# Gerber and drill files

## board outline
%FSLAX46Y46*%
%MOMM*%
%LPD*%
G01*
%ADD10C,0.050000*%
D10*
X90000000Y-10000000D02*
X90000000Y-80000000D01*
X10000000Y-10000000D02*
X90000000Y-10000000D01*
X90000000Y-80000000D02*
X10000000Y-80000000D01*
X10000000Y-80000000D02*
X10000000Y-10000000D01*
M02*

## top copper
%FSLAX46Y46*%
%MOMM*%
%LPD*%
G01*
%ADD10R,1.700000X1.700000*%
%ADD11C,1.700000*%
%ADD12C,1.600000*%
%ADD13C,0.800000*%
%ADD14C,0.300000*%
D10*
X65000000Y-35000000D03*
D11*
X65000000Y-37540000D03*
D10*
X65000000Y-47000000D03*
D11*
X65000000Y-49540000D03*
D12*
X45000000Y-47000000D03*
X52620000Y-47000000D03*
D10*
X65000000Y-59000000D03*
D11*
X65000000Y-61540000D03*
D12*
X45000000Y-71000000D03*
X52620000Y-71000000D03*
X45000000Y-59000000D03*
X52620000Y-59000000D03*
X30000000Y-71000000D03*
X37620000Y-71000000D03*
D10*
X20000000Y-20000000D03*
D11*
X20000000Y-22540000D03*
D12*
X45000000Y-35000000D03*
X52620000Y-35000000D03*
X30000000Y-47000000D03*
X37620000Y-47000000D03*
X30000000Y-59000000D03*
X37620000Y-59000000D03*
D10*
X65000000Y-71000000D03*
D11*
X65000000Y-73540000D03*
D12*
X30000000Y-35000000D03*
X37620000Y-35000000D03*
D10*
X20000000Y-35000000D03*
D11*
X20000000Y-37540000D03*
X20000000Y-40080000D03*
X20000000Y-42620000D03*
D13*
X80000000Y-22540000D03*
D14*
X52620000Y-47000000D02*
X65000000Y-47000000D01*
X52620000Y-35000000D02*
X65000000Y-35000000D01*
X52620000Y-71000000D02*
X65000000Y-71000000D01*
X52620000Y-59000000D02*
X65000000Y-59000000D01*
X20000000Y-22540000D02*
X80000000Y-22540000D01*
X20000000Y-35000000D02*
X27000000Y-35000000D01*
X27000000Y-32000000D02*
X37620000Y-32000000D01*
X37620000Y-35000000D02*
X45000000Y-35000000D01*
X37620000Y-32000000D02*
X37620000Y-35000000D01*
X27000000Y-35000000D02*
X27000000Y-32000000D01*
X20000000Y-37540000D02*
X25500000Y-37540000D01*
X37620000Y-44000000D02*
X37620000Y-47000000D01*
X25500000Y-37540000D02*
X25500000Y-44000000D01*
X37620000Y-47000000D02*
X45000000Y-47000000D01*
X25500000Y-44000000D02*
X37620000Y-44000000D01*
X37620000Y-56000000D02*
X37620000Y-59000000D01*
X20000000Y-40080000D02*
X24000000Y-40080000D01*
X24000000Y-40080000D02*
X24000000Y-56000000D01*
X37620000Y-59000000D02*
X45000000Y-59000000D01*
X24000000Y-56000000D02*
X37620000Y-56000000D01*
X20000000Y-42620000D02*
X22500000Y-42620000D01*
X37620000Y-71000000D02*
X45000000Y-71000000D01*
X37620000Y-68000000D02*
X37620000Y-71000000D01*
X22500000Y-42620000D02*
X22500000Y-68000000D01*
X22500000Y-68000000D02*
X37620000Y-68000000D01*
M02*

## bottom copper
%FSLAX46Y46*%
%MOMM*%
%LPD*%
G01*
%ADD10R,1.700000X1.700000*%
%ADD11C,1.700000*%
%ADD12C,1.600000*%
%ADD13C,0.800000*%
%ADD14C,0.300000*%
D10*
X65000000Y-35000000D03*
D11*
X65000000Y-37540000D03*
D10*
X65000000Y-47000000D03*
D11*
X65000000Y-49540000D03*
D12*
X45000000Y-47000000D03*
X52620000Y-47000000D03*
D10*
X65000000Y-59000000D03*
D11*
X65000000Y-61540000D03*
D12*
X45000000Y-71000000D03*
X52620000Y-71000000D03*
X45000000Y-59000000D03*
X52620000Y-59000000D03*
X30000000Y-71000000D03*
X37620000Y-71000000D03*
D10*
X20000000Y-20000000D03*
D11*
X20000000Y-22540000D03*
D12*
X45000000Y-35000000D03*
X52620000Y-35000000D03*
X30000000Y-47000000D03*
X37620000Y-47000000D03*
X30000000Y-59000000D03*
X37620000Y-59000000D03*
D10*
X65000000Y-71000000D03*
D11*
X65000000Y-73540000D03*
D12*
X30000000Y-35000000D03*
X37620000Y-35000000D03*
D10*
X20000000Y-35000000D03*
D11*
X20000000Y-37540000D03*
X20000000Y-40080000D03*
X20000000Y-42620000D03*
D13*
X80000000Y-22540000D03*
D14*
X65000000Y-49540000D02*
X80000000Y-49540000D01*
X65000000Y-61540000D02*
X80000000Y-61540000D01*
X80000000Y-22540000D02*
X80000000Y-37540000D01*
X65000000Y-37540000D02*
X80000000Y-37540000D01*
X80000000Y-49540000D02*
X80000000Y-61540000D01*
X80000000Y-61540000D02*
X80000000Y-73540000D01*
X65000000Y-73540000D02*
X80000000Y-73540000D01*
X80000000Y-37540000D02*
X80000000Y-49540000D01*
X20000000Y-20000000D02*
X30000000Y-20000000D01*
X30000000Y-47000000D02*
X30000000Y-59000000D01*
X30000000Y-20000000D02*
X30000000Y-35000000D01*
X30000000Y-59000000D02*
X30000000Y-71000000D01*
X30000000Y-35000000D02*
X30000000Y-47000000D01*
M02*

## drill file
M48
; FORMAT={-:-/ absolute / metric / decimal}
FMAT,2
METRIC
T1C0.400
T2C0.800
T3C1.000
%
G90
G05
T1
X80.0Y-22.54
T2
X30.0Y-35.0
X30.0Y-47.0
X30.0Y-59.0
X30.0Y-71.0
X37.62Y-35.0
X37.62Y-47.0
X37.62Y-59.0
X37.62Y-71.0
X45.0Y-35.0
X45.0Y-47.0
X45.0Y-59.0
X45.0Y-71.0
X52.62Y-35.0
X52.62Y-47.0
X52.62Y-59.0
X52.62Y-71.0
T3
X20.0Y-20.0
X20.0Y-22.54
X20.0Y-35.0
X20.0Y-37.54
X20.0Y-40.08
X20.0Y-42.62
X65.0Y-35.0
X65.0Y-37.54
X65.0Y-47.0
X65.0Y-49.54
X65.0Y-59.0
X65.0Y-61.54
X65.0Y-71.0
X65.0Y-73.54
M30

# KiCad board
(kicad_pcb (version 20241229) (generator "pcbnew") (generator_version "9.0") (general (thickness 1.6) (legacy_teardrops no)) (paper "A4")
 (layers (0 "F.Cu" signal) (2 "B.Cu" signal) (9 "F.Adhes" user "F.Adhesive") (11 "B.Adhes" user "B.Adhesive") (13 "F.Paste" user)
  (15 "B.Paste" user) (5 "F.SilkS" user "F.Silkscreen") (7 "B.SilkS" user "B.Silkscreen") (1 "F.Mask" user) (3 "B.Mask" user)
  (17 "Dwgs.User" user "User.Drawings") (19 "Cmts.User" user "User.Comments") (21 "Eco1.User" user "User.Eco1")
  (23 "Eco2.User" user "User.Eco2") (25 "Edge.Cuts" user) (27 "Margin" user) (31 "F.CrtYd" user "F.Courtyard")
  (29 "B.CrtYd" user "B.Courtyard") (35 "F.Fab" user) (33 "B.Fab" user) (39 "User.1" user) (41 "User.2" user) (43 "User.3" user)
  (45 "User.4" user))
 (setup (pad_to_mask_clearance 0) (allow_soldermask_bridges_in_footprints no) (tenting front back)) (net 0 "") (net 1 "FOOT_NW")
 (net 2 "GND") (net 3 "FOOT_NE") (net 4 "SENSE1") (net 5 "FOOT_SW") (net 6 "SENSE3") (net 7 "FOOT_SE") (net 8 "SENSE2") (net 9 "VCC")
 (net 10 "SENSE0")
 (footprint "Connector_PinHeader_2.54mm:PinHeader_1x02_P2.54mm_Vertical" (layer "F.Cu") (at 65 35)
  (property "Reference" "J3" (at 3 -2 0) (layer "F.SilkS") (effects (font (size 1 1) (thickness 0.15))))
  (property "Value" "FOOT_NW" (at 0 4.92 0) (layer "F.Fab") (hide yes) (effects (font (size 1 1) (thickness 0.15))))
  (pad "1" thru_hole rect (at 0 0) (size 1.7 1.7) (drill 1) (layers "*.Cu" "*.Mask") (remove_unused_layers no) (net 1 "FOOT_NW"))
  (pad "2" thru_hole circle (at 0 2.54) (size 1.7 1.7) (drill 1) (layers "*.Cu" "*.Mask") (remove_unused_layers no) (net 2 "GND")))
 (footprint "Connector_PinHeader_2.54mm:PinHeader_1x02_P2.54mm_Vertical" (layer "F.Cu") (at 65 47)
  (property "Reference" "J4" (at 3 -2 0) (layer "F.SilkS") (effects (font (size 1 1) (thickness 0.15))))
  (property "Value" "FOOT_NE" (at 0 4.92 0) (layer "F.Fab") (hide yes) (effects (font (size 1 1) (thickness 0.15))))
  (pad "1" thru_hole rect (at 0 0) (size 1.7 1.7) (drill 1) (layers "*.Cu" "*.Mask") (remove_unused_layers no) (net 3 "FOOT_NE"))
  (pad "2" thru_hole circle (at 0 2.54) (size 1.7 1.7) (drill 1) (layers "*.Cu" "*.Mask") (remove_unused_layers no) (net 2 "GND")))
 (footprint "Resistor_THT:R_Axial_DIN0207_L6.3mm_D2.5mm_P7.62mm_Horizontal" (layer "F.Cu") (at 45 47)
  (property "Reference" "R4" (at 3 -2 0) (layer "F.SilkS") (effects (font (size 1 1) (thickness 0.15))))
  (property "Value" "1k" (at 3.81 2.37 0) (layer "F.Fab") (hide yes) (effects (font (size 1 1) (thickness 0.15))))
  (pad "1" thru_hole circle (at 0 0) (size 1.6 1.6) (drill 0.8) (layers "*.Cu" "*.Mask") (remove_unused_layers no) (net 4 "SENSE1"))
  (pad "2" thru_hole circle (at 7.62 0) (size 1.6 1.6) (drill 0.8) (layers "*.Cu" "*.Mask") (remove_unused_layers no) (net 3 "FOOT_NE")))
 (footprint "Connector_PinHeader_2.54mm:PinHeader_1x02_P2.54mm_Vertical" (layer "F.Cu") (at 65 59)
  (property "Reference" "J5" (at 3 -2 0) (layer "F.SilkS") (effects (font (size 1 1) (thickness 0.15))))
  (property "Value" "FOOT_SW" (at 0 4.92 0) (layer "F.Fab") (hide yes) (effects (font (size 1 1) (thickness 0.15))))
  (pad "1" thru_hole rect (at 0 0) (size 1.7 1.7) (drill 1) (layers "*.Cu" "*.Mask") (remove_unused_layers no) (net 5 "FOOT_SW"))
  (pad "2" thru_hole circle (at 0 2.54) (size 1.7 1.7) (drill 1) (layers "*.Cu" "*.Mask") (remove_unused_layers no) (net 2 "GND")))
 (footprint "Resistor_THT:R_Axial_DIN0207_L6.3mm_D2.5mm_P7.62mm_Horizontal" (layer "F.Cu") (at 45 71)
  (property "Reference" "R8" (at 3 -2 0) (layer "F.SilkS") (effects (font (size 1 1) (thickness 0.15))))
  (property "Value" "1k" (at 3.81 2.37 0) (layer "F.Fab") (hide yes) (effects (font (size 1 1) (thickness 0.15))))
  (pad "1" thru_hole circle (at 0 0) (size 1.6 1.6) (drill 0.8) (layers "*.Cu" "*.Mask") (remove_unused_layers no) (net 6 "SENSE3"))
  (pad "2" thru_hole circle (at 7.62 0) (size 1.6 1.6) (drill 0.8) (layers "*.Cu" "*.Mask") (remove_unused_layers no) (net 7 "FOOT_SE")))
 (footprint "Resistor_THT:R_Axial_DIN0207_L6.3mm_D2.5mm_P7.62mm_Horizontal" (layer "F.Cu") (at 45 59)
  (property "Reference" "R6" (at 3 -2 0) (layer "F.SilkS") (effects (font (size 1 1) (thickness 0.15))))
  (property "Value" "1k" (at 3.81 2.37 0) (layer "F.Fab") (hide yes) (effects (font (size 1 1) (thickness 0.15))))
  (pad "1" thru_hole circle (at 0 0) (size 1.6 1.6) (drill 0.8) (layers "*.Cu" "*.Mask") (remove_unused_layers no) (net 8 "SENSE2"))
  (pad "2" thru_hole circle (at 7.62 0) (size 1.6 1.6) (drill 0.8) (layers "*.Cu" "*.Mask") (remove_unused_layers no) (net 5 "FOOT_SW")))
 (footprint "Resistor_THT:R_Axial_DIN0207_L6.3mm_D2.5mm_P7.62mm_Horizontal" (layer "F.Cu") (at 30 71)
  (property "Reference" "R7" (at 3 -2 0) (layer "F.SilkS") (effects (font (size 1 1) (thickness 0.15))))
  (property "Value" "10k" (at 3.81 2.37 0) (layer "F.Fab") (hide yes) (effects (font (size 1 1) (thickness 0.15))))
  (pad "1" thru_hole circle (at 0 0) (size 1.6 1.6) (drill 0.8) (layers "*.Cu" "*.Mask") (remove_unused_layers no) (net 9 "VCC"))
  (pad "2" thru_hole circle (at 7.62 0) (size 1.6 1.6) (drill 0.8) (layers "*.Cu" "*.Mask") (remove_unused_layers no) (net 6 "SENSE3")))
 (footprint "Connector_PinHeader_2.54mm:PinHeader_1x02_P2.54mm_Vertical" (layer "F.Cu") (at 20 20)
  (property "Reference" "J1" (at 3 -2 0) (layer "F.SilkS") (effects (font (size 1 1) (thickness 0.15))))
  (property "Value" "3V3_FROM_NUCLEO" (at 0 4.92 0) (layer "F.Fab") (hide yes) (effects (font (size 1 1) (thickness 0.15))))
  (pad "1" thru_hole rect (at 0 0) (size 1.7 1.7) (drill 1) (layers "*.Cu" "*.Mask") (remove_unused_layers no) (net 9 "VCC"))
  (pad "2" thru_hole circle (at 0 2.54) (size 1.7 1.7) (drill 1) (layers "*.Cu" "*.Mask") (remove_unused_layers no) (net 2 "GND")))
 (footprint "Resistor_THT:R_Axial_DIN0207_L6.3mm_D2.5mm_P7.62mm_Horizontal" (layer "F.Cu") (at 45 35)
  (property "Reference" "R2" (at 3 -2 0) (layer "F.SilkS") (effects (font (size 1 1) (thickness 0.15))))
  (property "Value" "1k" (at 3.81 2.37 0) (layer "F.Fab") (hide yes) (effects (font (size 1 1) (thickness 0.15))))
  (pad "1" thru_hole circle (at 0 0) (size 1.6 1.6) (drill 0.8) (layers "*.Cu" "*.Mask") (remove_unused_layers no) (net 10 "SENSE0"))
  (pad "2" thru_hole circle (at 7.62 0) (size 1.6 1.6) (drill 0.8) (layers "*.Cu" "*.Mask") (remove_unused_layers no) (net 1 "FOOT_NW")))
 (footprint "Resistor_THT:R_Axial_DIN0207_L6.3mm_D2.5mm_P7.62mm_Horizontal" (layer "F.Cu") (at 30 47)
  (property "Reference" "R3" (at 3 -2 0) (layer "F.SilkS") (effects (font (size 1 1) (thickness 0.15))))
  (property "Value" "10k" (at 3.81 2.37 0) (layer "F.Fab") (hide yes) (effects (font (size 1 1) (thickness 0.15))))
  (pad "1" thru_hole circle (at 0 0) (size 1.6 1.6) (drill 0.8) (layers "*.Cu" "*.Mask") (remove_unused_layers no) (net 9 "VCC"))
  (pad "2" thru_hole circle (at 7.62 0) (size 1.6 1.6) (drill 0.8) (layers "*.Cu" "*.Mask") (remove_unused_layers no) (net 4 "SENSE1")))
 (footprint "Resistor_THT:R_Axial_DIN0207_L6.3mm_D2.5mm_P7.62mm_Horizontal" (layer "F.Cu") (at 30 59)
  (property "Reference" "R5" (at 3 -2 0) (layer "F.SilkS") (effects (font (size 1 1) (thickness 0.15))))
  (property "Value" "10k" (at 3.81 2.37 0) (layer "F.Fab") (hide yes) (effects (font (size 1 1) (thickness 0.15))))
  (pad "1" thru_hole circle (at 0 0) (size 1.6 1.6) (drill 0.8) (layers "*.Cu" "*.Mask") (remove_unused_layers no) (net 9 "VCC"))
  (pad "2" thru_hole circle (at 7.62 0) (size 1.6 1.6) (drill 0.8) (layers "*.Cu" "*.Mask") (remove_unused_layers no) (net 8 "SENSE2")))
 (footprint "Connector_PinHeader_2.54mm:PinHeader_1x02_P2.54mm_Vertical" (layer "F.Cu") (at 65 71)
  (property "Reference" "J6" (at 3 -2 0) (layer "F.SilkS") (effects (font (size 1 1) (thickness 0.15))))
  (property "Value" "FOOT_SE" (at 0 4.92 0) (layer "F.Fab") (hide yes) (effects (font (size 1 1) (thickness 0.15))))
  (pad "1" thru_hole rect (at 0 0) (size 1.7 1.7) (drill 1) (layers "*.Cu" "*.Mask") (remove_unused_layers no) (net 7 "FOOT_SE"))
  (pad "2" thru_hole circle (at 0 2.54) (size 1.7 1.7) (drill 1) (layers "*.Cu" "*.Mask") (remove_unused_layers no) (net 2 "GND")))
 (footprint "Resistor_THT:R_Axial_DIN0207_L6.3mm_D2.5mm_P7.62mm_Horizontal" (layer "F.Cu") (at 30 35)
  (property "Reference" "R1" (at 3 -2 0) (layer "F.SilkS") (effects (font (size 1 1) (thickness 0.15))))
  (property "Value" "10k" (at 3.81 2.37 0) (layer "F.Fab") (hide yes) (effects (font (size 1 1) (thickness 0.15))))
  (pad "1" thru_hole circle (at 0 0) (size 1.6 1.6) (drill 0.8) (layers "*.Cu" "*.Mask") (remove_unused_layers no) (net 9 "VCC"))
  (pad "2" thru_hole circle (at 7.62 0) (size 1.6 1.6) (drill 0.8) (layers "*.Cu" "*.Mask") (remove_unused_layers no) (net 10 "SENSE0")))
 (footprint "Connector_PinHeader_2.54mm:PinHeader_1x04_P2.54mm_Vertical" (layer "F.Cu") (at 20 35)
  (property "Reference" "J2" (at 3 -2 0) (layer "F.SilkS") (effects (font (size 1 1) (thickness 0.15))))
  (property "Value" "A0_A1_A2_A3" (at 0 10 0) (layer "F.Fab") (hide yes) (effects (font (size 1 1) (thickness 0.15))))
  (pad "1" thru_hole rect (at 0 0) (size 1.7 1.7) (drill 1) (layers "*.Cu" "*.Mask") (remove_unused_layers no) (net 10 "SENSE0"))
  (pad "2" thru_hole circle (at 0 2.54) (size 1.7 1.7) (drill 1) (layers "*.Cu" "*.Mask") (remove_unused_layers no) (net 4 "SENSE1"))
  (pad "3" thru_hole circle (at 0 5.08) (size 1.7 1.7) (drill 1) (layers "*.Cu" "*.Mask") (remove_unused_layers no) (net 8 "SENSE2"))
  (pad "4" thru_hole circle (at 0 7.62) (size 1.7 1.7) (drill 1) (layers "*.Cu" "*.Mask") (remove_unused_layers no) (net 6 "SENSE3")))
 (gr_line (start 90 10) (end 90 80) (stroke (width 0.05) (type default)) (layer "Edge.Cuts"))
 (gr_line (start 10 10) (end 90 10) (stroke (width 0.05) (type default)) (layer "Edge.Cuts"))
 (gr_line (start 90 80) (end 10 80) (stroke (width 0.05) (type default)) (layer "Edge.Cuts"))
 (gr_line (start 10 80) (end 10 10) (stroke (width 0.05) (type default)) (layer "Edge.Cuts"))
 (segment (start 52.62 47) (end 65 47) (width 0.3) (layer "F.Cu") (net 3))
 (segment (start 52.62 35) (end 65 35) (width 0.3) (layer "F.Cu") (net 1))
 (segment (start 52.62 71) (end 65 71) (width 0.3) (layer "F.Cu") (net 7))
 (segment (start 52.62 59) (end 65 59) (width 0.3) (layer "F.Cu") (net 5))
 (segment (start 20 22.54) (end 80 22.54) (width 0.3) (layer "F.Cu") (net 2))
 (via (at 80 22.54) (size 0.8) (drill 0.4) (layers "F.Cu" "B.Cu") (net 2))
 (segment (start 65 49.54) (end 80 49.54) (width 0.3) (layer "B.Cu") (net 2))
 (segment (start 65 61.54) (end 80 61.54) (width 0.3) (layer "B.Cu") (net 2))
 (segment (start 80 22.54) (end 80 37.54) (width 0.3) (layer "B.Cu") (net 2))
 (segment (start 65 37.54) (end 80 37.54) (width 0.3) (layer "B.Cu") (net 2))
 (segment (start 80 49.54) (end 80 61.54) (width 0.3) (layer "B.Cu") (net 2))
 (segment (start 80 61.54) (end 80 73.54) (width 0.3) (layer "B.Cu") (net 2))
 (segment (start 65 73.54) (end 80 73.54) (width 0.3) (layer "B.Cu") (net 2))
 (segment (start 80 37.54) (end 80 49.54) (width 0.3) (layer "B.Cu") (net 2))
 (segment (start 20 35) (end 27 35) (width 0.3) (layer "F.Cu") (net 10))
 (segment (start 27 32) (end 37.62 32) (width 0.3) (layer "F.Cu") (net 10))
 (segment (start 37.62 35) (end 45 35) (width 0.3) (layer "F.Cu") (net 10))
 (segment (start 37.62 32) (end 37.62 35) (width 0.3) (layer "F.Cu") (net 10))
 (segment (start 27 35) (end 27 32) (width 0.3) (layer "F.Cu") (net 10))
 (segment (start 20 37.54) (end 25.5 37.54) (width 0.3) (layer "F.Cu") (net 4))
 (segment (start 37.62 44) (end 37.62 47) (width 0.3) (layer "F.Cu") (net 4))
 (segment (start 25.5 37.54) (end 25.5 44) (width 0.3) (layer "F.Cu") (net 4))
 (segment (start 37.62 47) (end 45 47) (width 0.3) (layer "F.Cu") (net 4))
 (segment (start 25.5 44) (end 37.62 44) (width 0.3) (layer "F.Cu") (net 4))
 (segment (start 37.62 56) (end 37.62 59) (width 0.3) (layer "F.Cu") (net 8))
 (segment (start 20 40.08) (end 24 40.08) (width 0.3) (layer "F.Cu") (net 8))
 (segment (start 24 40.08) (end 24 56) (width 0.3) (layer "F.Cu") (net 8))
 (segment (start 37.62 59) (end 45 59) (width 0.3) (layer "F.Cu") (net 8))
 (segment (start 24 56) (end 37.62 56) (width 0.3) (layer "F.Cu") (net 8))
 (segment (start 20 42.62) (end 22.5 42.62) (width 0.3) (layer "F.Cu") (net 6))
 (segment (start 37.62 71) (end 45 71) (width 0.3) (layer "F.Cu") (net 6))
 (segment (start 37.62 68) (end 37.62 71) (width 0.3) (layer "F.Cu") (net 6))
 (segment (start 22.5 42.62) (end 22.5 68) (width 0.3) (layer "F.Cu") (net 6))
 (segment (start 22.5 68) (end 37.62 68) (width 0.3) (layer "F.Cu") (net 6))
 (segment (start 20 20) (end 30 20) (width 0.3) (layer "B.Cu") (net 9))
 (segment (start 30 47) (end 30 59) (width 0.3) (layer "B.Cu") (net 9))
 (segment (start 30 20) (end 30 35) (width 0.3) (layer "B.Cu") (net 9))
 (segment (start 30 59) (end 30 71) (width 0.3) (layer "B.Cu") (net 9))
 (segment (start 30 35) (end 30 47) (width 0.3) (layer "B.Cu") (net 9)))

